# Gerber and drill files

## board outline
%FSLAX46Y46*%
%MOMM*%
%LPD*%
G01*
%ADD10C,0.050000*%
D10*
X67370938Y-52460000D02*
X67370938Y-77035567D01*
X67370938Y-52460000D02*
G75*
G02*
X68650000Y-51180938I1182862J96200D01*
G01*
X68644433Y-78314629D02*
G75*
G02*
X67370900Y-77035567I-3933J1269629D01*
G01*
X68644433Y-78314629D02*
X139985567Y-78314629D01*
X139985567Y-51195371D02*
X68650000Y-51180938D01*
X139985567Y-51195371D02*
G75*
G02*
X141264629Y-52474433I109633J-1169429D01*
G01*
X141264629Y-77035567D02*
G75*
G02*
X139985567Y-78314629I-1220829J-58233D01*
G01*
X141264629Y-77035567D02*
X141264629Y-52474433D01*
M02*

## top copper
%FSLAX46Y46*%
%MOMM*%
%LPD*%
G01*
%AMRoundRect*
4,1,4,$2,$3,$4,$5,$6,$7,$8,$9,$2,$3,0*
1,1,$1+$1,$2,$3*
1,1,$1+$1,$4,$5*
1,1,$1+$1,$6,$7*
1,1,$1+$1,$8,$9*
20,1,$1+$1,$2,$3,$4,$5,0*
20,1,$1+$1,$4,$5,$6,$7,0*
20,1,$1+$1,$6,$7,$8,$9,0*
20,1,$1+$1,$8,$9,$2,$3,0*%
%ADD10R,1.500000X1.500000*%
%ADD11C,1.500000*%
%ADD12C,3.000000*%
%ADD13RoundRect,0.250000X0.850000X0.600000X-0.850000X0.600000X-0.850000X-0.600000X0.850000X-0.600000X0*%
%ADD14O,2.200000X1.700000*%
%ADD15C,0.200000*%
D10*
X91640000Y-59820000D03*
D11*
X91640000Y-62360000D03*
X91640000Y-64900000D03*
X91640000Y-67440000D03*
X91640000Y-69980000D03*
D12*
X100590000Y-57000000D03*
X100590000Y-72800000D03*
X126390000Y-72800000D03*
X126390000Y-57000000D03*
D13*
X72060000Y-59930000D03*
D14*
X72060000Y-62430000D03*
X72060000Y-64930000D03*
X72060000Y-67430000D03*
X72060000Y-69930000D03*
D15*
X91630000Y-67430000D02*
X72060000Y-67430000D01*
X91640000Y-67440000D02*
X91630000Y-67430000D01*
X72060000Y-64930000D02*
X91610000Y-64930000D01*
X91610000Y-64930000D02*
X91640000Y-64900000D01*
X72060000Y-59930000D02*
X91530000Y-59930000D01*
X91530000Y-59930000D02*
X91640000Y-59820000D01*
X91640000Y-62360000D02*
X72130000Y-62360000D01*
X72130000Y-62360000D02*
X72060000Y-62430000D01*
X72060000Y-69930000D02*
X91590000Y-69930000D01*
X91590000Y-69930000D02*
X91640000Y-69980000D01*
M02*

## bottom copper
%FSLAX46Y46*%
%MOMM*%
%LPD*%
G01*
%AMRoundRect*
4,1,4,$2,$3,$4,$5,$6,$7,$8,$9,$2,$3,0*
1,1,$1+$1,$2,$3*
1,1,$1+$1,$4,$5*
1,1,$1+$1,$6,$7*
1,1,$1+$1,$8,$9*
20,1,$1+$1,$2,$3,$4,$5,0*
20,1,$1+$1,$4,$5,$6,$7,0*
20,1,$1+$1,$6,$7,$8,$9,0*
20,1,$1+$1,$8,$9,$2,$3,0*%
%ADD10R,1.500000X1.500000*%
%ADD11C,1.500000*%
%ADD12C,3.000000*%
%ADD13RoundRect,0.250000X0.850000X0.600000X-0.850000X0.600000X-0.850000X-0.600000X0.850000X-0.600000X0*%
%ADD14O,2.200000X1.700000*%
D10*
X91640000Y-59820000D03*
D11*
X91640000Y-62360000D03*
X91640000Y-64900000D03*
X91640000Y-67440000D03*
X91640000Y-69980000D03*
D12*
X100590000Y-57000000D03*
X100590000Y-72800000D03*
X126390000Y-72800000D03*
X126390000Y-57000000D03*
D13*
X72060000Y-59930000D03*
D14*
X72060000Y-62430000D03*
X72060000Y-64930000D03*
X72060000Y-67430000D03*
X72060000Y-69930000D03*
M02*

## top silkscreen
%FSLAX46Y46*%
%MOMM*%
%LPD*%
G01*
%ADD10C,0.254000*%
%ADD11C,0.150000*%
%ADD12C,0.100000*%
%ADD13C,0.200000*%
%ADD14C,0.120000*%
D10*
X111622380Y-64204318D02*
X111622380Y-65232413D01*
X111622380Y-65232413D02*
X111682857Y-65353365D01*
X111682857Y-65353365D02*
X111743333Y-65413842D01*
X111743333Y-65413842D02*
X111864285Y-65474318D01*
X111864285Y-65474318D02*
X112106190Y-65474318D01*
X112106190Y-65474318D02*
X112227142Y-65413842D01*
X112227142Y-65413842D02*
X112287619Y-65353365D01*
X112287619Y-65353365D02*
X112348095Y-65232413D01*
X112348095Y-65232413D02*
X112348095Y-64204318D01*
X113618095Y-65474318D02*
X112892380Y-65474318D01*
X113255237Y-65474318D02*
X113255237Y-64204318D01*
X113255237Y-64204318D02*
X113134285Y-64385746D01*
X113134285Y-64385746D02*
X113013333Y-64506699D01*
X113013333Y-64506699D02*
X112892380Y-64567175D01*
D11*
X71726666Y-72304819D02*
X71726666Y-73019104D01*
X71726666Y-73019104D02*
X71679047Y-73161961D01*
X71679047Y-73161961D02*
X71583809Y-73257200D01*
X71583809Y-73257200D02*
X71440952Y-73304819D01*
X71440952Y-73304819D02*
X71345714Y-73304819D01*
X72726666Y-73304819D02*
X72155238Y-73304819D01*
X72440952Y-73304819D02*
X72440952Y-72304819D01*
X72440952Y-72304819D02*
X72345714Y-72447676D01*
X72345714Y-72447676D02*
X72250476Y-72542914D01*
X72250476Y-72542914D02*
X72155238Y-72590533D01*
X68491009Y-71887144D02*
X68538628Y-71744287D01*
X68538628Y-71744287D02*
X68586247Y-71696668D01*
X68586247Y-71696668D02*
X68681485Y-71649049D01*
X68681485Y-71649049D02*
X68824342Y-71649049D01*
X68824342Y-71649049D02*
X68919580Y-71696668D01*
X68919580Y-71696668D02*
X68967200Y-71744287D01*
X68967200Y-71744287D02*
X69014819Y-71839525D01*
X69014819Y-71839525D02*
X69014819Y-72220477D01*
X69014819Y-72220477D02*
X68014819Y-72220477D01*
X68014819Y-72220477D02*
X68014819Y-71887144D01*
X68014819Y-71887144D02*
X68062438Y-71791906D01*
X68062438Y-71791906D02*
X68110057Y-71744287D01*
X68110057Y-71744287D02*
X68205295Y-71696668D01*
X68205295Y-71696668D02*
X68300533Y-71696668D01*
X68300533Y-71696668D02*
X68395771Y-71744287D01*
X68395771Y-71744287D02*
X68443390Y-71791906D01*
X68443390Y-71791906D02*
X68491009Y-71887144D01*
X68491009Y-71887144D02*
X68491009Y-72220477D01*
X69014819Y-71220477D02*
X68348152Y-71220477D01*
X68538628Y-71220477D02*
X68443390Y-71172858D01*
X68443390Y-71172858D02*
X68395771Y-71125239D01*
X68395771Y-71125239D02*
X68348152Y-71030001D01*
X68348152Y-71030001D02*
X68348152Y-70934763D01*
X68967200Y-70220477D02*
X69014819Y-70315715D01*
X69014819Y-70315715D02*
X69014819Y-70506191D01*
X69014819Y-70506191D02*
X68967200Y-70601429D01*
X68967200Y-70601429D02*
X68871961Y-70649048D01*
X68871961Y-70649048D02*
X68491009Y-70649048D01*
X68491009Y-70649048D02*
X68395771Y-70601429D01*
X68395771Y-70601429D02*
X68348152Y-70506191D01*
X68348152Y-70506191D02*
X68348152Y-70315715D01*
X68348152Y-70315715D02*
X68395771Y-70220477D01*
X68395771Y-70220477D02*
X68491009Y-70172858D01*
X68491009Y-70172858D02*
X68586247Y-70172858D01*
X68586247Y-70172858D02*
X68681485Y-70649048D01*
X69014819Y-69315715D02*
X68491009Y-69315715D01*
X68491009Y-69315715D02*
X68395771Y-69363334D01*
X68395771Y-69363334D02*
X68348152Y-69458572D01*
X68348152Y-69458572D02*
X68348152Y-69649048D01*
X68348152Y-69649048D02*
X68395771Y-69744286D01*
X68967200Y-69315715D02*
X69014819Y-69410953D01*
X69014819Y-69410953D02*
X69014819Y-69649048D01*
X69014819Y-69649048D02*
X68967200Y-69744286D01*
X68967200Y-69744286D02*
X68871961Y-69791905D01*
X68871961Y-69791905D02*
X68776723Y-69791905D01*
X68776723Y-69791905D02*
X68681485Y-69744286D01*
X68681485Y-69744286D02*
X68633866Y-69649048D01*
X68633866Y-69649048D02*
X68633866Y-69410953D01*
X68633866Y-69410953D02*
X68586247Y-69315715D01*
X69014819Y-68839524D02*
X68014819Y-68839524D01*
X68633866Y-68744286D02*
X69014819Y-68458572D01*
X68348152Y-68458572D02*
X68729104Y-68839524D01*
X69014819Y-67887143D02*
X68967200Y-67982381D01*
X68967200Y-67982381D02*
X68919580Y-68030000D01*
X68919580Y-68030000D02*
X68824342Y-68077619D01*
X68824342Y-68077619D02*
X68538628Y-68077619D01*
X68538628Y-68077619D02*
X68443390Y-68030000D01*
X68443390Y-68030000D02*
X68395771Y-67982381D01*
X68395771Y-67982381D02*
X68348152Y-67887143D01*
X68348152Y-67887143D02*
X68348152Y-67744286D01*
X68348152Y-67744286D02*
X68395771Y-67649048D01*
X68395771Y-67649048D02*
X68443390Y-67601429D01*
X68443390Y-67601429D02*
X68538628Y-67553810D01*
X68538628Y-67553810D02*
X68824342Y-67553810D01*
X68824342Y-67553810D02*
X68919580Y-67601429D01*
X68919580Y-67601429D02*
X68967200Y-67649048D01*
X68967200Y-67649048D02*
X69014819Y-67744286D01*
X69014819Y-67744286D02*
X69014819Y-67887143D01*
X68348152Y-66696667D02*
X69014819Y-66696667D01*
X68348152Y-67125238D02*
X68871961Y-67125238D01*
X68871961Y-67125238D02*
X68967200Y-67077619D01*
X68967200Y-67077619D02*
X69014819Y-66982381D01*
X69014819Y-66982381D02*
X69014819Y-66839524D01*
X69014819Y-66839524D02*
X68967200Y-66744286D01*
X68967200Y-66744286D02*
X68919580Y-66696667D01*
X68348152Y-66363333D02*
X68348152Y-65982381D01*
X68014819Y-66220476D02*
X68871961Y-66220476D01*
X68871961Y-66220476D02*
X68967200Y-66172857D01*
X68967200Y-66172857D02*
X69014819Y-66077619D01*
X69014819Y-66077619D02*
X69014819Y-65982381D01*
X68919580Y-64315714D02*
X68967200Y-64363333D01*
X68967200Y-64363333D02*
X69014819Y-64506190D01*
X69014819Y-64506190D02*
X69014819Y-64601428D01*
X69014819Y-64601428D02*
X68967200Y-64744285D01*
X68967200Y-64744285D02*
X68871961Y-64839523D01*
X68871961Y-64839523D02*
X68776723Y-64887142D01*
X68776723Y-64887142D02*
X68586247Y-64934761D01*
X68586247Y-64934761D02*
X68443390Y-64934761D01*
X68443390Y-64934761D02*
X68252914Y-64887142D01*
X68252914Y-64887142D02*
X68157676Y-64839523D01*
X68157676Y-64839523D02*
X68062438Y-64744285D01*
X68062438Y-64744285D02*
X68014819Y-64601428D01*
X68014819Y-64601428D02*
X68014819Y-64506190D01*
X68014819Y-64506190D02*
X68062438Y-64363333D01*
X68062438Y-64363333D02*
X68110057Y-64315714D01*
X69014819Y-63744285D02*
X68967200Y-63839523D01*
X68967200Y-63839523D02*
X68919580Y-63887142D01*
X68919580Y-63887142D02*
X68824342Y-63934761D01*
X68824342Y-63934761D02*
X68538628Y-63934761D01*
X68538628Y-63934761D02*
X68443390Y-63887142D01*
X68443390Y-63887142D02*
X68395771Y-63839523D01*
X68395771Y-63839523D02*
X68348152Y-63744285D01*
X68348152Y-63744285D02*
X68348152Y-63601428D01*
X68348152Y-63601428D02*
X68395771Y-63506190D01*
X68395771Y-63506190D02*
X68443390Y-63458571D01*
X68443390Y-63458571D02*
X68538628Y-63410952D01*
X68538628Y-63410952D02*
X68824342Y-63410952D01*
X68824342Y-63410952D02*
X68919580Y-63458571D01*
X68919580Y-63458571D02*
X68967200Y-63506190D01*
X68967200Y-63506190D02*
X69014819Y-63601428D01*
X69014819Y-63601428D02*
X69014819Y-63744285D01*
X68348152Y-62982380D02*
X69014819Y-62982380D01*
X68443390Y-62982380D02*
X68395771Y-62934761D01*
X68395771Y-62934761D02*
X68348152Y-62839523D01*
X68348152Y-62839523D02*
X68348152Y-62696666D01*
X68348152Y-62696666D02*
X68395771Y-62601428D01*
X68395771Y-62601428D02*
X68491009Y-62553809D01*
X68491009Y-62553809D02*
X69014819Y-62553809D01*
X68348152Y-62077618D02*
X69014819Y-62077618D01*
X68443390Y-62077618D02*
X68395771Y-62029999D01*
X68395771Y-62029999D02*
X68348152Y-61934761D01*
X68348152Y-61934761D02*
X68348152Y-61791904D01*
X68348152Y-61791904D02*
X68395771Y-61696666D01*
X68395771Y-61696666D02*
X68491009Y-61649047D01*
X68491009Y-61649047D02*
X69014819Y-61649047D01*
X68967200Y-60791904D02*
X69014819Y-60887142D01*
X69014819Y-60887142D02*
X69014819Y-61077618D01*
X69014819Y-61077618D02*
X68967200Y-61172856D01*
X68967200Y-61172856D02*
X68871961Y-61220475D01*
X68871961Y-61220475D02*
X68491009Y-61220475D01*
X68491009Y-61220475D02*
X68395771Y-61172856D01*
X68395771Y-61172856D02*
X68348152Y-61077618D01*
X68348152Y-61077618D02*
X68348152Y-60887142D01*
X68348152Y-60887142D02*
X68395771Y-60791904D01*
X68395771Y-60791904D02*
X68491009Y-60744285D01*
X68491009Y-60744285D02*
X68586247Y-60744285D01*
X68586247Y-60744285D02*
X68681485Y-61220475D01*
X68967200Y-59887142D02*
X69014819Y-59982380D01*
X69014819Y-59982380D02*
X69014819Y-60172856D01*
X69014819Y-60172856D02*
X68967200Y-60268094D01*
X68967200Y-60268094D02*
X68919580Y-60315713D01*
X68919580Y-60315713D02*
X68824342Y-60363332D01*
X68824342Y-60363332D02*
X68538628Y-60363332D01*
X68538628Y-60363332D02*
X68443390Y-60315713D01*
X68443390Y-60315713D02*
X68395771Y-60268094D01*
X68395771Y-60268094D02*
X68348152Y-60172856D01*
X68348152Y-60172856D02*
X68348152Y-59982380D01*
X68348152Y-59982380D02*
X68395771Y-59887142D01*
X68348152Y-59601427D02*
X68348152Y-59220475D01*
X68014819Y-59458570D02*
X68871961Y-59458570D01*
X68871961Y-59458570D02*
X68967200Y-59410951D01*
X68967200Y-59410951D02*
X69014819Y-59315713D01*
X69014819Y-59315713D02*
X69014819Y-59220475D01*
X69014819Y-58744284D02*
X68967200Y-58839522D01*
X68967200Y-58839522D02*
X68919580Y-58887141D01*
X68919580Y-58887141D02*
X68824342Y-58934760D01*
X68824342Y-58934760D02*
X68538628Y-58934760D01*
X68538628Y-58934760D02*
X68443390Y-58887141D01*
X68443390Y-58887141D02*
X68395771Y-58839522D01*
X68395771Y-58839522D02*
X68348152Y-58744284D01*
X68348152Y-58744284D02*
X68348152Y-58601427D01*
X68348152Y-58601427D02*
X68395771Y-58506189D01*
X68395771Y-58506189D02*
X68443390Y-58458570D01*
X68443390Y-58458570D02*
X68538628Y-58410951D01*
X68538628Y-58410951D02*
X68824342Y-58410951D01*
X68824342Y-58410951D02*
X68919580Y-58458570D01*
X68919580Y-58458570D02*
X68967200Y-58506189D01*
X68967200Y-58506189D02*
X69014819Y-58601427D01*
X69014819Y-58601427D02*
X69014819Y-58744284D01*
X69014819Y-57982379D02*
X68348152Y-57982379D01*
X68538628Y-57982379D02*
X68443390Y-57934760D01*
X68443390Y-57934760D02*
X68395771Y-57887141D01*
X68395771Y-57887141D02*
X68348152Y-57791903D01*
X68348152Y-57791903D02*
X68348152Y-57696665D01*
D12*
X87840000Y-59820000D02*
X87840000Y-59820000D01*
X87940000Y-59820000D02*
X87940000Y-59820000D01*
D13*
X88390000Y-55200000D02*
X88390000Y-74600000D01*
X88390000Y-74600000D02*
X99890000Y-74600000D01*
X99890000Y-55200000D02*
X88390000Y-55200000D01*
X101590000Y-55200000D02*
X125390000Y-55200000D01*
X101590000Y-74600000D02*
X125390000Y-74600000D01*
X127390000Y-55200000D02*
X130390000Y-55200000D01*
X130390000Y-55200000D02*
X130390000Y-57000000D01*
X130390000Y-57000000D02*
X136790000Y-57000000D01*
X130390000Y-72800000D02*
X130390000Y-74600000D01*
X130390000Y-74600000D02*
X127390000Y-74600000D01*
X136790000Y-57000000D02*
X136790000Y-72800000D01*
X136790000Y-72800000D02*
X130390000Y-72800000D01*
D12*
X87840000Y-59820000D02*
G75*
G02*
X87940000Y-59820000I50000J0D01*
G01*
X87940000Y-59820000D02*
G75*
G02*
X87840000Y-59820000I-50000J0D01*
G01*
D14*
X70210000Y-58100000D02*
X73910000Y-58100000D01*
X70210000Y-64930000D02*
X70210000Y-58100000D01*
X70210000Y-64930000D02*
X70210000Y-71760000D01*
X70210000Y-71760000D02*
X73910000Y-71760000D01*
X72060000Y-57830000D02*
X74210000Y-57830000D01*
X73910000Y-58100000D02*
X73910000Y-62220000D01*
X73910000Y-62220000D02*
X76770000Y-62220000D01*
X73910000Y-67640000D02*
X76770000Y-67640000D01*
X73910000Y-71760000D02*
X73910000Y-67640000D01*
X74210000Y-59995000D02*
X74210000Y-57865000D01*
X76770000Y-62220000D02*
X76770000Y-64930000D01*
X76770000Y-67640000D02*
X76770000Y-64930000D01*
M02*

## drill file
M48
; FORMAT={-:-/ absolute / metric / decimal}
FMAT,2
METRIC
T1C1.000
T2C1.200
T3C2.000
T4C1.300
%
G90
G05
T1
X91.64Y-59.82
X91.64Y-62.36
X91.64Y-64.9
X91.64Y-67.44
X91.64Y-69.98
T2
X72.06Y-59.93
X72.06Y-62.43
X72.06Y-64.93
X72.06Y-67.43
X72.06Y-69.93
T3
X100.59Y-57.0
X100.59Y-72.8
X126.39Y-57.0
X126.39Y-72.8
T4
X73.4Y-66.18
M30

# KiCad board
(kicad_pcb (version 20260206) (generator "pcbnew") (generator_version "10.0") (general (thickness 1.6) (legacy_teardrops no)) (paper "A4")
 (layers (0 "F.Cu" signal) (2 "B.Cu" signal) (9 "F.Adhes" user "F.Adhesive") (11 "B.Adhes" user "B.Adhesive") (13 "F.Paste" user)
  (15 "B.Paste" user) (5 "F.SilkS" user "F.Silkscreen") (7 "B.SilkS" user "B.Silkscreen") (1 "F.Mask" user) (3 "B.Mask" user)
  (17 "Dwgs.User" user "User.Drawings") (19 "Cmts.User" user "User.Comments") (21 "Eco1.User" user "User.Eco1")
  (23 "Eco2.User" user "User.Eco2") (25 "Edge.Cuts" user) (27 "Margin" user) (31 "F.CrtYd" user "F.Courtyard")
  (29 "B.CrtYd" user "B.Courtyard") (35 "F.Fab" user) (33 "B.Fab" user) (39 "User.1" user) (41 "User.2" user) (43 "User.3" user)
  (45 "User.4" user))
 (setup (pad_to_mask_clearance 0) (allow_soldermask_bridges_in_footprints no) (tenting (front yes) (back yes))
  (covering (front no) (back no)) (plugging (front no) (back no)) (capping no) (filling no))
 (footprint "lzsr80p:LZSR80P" (layer "F.Cu") (at 91.64 59.82)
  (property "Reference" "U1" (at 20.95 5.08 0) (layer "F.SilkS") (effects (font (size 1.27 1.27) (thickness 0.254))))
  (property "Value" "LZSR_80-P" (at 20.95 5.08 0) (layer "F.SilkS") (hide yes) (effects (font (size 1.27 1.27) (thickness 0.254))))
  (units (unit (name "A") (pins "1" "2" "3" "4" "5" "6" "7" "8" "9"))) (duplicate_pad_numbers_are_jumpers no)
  (fp_line (start -3.8 0) (end -3.8 0) (stroke (width 0.1) (type solid)) (layer "F.SilkS"))
  (fp_line (start -3.7 0) (end -3.7 0) (stroke (width 0.1) (type solid)) (layer "F.SilkS"))
  (fp_line (start -3.25 -4.62) (end -3.25 14.78) (stroke (width 0.2) (type solid)) (layer "F.SilkS"))
  (fp_line (start -3.25 14.78) (end 8.25 14.78) (stroke (width 0.2) (type solid)) (layer "F.SilkS"))
  (fp_line (start 8.25 -4.62) (end -3.25 -4.62) (stroke (width 0.2) (type solid)) (layer "F.SilkS"))
  (fp_line (start 9.95 -4.62) (end 33.75 -4.62) (stroke (width 0.2) (type solid)) (layer "F.SilkS"))
  (fp_line (start 9.95 14.78) (end 33.75 14.78) (stroke (width 0.2) (type solid)) (layer "F.SilkS"))
  (fp_line (start 35.75 -4.62) (end 38.75 -4.62) (stroke (width 0.2) (type solid)) (layer "F.SilkS"))
  (fp_line (start 38.75 -4.62) (end 38.75 -2.82) (stroke (width 0.2) (type solid)) (layer "F.SilkS"))
  (fp_line (start 38.75 -2.82) (end 45.15 -2.82) (stroke (width 0.2) (type solid)) (layer "F.SilkS"))
  (fp_line (start 38.75 12.98) (end 38.75 14.78) (stroke (width 0.2) (type solid)) (layer "F.SilkS"))
  (fp_line (start 38.75 14.78) (end 35.75 14.78) (stroke (width 0.2) (type solid)) (layer "F.SilkS"))
  (fp_line (start 45.15 -2.82) (end 45.15 12.98) (stroke (width 0.2) (type solid)) (layer "F.SilkS"))
  (fp_line (start 45.15 12.98) (end 38.75 12.98) (stroke (width 0.2) (type solid)) (layer "F.SilkS"))
  (fp_arc (start -3.8 0) (mid -3.75 -0.05) (end -3.7 0) (stroke (width 0.1) (type solid)) (layer "F.SilkS"))
  (fp_arc (start -3.7 0) (mid -3.75 0.05) (end -3.8 0) (stroke (width 0.1) (type solid)) (layer "F.SilkS"))
  (pad "1" thru_hole rect (at 0 0) (size 1.5 1.5) (drill 1) (layers "*.Cu" "*.Mask") (remove_unused_layers no) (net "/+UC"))
  (pad "2" thru_hole circle (at 0 2.54) (size 1.5 1.5) (drill 1) (layers "*.Cu" "*.Mask") (remove_unused_layers no) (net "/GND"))
  (pad "3" thru_hole circle (at 0 5.08) (size 1.5 1.5) (drill 1) (layers "*.Cu" "*.Mask") (remove_unused_layers no) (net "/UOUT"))
  (pad "4" thru_hole circle (at 0 7.62) (size 1.5 1.5) (drill 1) (layers "*.Cu" "*.Mask") (remove_unused_layers no) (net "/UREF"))
  (pad "5" thru_hole circle (at 0 10.16) (size 1.5 1.5) (drill 1) (layers "*.Cu" "*.Mask") (remove_unused_layers no) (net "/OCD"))
  (pad "6" thru_hole circle (at 8.95 -2.82) (size 3 3) (drill 2) (layers "*.Cu" "*.Mask") (remove_unused_layers no)
   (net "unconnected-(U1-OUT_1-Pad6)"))
  (pad "7" thru_hole circle (at 8.95 12.98) (size 3 3) (drill 2) (layers "*.Cu" "*.Mask") (remove_unused_layers no)
   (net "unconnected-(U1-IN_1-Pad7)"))
  (pad "8" thru_hole circle (at 34.75 12.98) (size 3 3) (drill 2) (layers "*.Cu" "*.Mask") (remove_unused_layers no)
   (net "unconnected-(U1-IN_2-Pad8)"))
  (pad "9" thru_hole circle (at 34.75 -2.82) (size 3 3) (drill 2) (layers "*.Cu" "*.Mask") (remove_unused_layers no)
   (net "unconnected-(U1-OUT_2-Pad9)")))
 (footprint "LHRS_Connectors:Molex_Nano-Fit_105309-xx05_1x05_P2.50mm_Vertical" (layer "F.Cu") (at 72.06 69.93 180)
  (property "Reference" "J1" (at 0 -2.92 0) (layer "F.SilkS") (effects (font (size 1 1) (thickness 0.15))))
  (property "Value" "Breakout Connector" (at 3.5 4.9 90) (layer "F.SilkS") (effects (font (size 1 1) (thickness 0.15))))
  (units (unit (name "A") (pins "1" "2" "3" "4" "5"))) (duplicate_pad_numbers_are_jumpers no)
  (fp_line (start 1.85 11.83) (end -1.85 11.83) (stroke (width 0.12) (type solid)) (layer "F.SilkS"))
  (fp_line (start 1.85 5) (end 1.85 11.83) (stroke (width 0.12) (type solid)) (layer "F.SilkS"))
  (fp_line (start 1.85 5) (end 1.85 -1.83) (stroke (width 0.12) (type solid)) (layer "F.SilkS"))
  (fp_line (start 1.85 -1.83) (end -1.85 -1.83) (stroke (width 0.12) (type solid)) (layer "F.SilkS"))
  (fp_line (start 0 12.1) (end -2.15 12.1) (stroke (width 0.12) (type solid)) (layer "F.SilkS"))
  (fp_line (start -1.85 11.83) (end -1.85 7.71) (stroke (width 0.12) (type solid)) (layer "F.SilkS"))
  (fp_line (start -1.85 7.71) (end -4.71 7.71) (stroke (width 0.12) (type solid)) (layer "F.SilkS"))
  (fp_line (start -1.85 2.29) (end -4.71 2.29) (stroke (width 0.12) (type solid)) (layer "F.SilkS"))
  (fp_line (start -1.85 -1.83) (end -1.85 2.29) (stroke (width 0.12) (type solid)) (layer "F.SilkS"))
  (fp_line (start -2.15 9.935) (end -2.15 12.065) (stroke (width 0.12) (type solid)) (layer "F.SilkS"))
  (fp_line (start -4.71 7.71) (end -4.71 5) (stroke (width 0.12) (type solid)) (layer "F.SilkS"))
  (fp_line (start -4.71 2.29) (end -4.71 5) (stroke (width 0.12) (type solid)) (layer "F.SilkS"))
  (pad "" np_thru_hole circle (at -1.34 3.75 180) (size 1.3 1.3) (drill 1.3) (layers "*.Cu" "*.Mask"))
  (pad "1" thru_hole roundrect (at 0 10 180) (size 2.2 1.7) (drill 1.2) (layers "*.Cu" "*.Mask") (remove_unused_layers no)
   (roundrect_rratio 0.1470588235) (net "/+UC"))
  (pad "2" thru_hole oval (at 0 7.5 180) (size 2.2 1.7) (drill 1.2) (layers "*.Cu" "*.Mask") (remove_unused_layers no) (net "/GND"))
  (pad "3" thru_hole oval (at 0 5 180) (size 2.2 1.7) (drill 1.2) (layers "*.Cu" "*.Mask") (remove_unused_layers no) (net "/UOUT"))
  (pad "4" thru_hole oval (at 0 2.5 180) (size 2.2 1.7) (drill 1.2) (layers "*.Cu" "*.Mask") (remove_unused_layers no) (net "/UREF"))
  (pad "5" thru_hole oval (at 0 0 180) (size 2.2 1.7) (drill 1.2) (layers "*.Cu" "*.Mask") (remove_unused_layers no) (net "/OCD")))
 (gr_line (start 67.370938 52.46) (end 67.370938 77.035567) (stroke (width 0.05) (type default)) (layer "Edge.Cuts"))
 (gr_arc (start 67.370938 52.46) (mid 67.74 51.5) (end 68.65 51.180938) (stroke (width 0.05) (type solid)) (layer "Edge.Cuts"))
 (gr_arc (start 68.644433 78.314629) (mid 67.74 77.94) (end 67.370938 77.035567) (stroke (width 0.05) (type solid)) (layer "Edge.Cuts"))
 (gr_line (start 68.644433 78.314629) (end 139.985567 78.314629) (stroke (width 0.05) (type default)) (layer "Edge.Cuts"))
 (gr_line (start 139.985567 51.195371) (end 68.65 51.180938) (stroke (width 0.05) (type default)) (layer "Edge.Cuts"))
 (gr_arc (start 139.985567 51.195371) (mid 140.925737 51.534263) (end 141.264629 52.474433) (stroke (width 0.05) (type solid))
  (layer "Edge.Cuts"))
 (gr_arc (start 141.264629 77.035567) (mid 140.925737 77.94) (end 139.985567 78.314629) (stroke (width 0.05) (type solid))
  (layer "Edge.Cuts"))
 (gr_line (start 141.264629 77.035567) (end 141.264629 52.474433) (stroke (width 0.05) (type default)) (layer "Edge.Cuts"))
 (segment (start 91.63 67.43) (end 72.06 67.43) (width 0.2) (layer "F.Cu") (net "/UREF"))
 (segment (start 91.64 67.44) (end 91.63 67.43) (width 0.2) (layer "F.Cu") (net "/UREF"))
 (segment (start 72.06 64.93) (end 91.61 64.93) (width 0.2) (layer "F.Cu") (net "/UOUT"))
 (segment (start 91.61 64.93) (end 91.64 64.9) (width 0.2) (layer "F.Cu") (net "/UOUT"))
 (segment (start 72.06 59.93) (end 91.53 59.93) (width 0.2) (layer "F.Cu") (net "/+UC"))
 (segment (start 91.53 59.93) (end 91.64 59.82) (width 0.2) (layer "F.Cu") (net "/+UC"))
 (segment (start 91.64 62.36) (end 72.13 62.36) (width 0.2) (layer "F.Cu") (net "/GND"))
 (segment (start 72.13 62.36) (end 72.06 62.43) (width 0.2) (layer "F.Cu") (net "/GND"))
 (segment (start 72.06 69.93) (end 91.59 69.93) (width 0.2) (layer "F.Cu") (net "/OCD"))
 (segment (start 91.59 69.93) (end 91.64 69.98) (width 0.2) (layer "F.Cu") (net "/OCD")))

